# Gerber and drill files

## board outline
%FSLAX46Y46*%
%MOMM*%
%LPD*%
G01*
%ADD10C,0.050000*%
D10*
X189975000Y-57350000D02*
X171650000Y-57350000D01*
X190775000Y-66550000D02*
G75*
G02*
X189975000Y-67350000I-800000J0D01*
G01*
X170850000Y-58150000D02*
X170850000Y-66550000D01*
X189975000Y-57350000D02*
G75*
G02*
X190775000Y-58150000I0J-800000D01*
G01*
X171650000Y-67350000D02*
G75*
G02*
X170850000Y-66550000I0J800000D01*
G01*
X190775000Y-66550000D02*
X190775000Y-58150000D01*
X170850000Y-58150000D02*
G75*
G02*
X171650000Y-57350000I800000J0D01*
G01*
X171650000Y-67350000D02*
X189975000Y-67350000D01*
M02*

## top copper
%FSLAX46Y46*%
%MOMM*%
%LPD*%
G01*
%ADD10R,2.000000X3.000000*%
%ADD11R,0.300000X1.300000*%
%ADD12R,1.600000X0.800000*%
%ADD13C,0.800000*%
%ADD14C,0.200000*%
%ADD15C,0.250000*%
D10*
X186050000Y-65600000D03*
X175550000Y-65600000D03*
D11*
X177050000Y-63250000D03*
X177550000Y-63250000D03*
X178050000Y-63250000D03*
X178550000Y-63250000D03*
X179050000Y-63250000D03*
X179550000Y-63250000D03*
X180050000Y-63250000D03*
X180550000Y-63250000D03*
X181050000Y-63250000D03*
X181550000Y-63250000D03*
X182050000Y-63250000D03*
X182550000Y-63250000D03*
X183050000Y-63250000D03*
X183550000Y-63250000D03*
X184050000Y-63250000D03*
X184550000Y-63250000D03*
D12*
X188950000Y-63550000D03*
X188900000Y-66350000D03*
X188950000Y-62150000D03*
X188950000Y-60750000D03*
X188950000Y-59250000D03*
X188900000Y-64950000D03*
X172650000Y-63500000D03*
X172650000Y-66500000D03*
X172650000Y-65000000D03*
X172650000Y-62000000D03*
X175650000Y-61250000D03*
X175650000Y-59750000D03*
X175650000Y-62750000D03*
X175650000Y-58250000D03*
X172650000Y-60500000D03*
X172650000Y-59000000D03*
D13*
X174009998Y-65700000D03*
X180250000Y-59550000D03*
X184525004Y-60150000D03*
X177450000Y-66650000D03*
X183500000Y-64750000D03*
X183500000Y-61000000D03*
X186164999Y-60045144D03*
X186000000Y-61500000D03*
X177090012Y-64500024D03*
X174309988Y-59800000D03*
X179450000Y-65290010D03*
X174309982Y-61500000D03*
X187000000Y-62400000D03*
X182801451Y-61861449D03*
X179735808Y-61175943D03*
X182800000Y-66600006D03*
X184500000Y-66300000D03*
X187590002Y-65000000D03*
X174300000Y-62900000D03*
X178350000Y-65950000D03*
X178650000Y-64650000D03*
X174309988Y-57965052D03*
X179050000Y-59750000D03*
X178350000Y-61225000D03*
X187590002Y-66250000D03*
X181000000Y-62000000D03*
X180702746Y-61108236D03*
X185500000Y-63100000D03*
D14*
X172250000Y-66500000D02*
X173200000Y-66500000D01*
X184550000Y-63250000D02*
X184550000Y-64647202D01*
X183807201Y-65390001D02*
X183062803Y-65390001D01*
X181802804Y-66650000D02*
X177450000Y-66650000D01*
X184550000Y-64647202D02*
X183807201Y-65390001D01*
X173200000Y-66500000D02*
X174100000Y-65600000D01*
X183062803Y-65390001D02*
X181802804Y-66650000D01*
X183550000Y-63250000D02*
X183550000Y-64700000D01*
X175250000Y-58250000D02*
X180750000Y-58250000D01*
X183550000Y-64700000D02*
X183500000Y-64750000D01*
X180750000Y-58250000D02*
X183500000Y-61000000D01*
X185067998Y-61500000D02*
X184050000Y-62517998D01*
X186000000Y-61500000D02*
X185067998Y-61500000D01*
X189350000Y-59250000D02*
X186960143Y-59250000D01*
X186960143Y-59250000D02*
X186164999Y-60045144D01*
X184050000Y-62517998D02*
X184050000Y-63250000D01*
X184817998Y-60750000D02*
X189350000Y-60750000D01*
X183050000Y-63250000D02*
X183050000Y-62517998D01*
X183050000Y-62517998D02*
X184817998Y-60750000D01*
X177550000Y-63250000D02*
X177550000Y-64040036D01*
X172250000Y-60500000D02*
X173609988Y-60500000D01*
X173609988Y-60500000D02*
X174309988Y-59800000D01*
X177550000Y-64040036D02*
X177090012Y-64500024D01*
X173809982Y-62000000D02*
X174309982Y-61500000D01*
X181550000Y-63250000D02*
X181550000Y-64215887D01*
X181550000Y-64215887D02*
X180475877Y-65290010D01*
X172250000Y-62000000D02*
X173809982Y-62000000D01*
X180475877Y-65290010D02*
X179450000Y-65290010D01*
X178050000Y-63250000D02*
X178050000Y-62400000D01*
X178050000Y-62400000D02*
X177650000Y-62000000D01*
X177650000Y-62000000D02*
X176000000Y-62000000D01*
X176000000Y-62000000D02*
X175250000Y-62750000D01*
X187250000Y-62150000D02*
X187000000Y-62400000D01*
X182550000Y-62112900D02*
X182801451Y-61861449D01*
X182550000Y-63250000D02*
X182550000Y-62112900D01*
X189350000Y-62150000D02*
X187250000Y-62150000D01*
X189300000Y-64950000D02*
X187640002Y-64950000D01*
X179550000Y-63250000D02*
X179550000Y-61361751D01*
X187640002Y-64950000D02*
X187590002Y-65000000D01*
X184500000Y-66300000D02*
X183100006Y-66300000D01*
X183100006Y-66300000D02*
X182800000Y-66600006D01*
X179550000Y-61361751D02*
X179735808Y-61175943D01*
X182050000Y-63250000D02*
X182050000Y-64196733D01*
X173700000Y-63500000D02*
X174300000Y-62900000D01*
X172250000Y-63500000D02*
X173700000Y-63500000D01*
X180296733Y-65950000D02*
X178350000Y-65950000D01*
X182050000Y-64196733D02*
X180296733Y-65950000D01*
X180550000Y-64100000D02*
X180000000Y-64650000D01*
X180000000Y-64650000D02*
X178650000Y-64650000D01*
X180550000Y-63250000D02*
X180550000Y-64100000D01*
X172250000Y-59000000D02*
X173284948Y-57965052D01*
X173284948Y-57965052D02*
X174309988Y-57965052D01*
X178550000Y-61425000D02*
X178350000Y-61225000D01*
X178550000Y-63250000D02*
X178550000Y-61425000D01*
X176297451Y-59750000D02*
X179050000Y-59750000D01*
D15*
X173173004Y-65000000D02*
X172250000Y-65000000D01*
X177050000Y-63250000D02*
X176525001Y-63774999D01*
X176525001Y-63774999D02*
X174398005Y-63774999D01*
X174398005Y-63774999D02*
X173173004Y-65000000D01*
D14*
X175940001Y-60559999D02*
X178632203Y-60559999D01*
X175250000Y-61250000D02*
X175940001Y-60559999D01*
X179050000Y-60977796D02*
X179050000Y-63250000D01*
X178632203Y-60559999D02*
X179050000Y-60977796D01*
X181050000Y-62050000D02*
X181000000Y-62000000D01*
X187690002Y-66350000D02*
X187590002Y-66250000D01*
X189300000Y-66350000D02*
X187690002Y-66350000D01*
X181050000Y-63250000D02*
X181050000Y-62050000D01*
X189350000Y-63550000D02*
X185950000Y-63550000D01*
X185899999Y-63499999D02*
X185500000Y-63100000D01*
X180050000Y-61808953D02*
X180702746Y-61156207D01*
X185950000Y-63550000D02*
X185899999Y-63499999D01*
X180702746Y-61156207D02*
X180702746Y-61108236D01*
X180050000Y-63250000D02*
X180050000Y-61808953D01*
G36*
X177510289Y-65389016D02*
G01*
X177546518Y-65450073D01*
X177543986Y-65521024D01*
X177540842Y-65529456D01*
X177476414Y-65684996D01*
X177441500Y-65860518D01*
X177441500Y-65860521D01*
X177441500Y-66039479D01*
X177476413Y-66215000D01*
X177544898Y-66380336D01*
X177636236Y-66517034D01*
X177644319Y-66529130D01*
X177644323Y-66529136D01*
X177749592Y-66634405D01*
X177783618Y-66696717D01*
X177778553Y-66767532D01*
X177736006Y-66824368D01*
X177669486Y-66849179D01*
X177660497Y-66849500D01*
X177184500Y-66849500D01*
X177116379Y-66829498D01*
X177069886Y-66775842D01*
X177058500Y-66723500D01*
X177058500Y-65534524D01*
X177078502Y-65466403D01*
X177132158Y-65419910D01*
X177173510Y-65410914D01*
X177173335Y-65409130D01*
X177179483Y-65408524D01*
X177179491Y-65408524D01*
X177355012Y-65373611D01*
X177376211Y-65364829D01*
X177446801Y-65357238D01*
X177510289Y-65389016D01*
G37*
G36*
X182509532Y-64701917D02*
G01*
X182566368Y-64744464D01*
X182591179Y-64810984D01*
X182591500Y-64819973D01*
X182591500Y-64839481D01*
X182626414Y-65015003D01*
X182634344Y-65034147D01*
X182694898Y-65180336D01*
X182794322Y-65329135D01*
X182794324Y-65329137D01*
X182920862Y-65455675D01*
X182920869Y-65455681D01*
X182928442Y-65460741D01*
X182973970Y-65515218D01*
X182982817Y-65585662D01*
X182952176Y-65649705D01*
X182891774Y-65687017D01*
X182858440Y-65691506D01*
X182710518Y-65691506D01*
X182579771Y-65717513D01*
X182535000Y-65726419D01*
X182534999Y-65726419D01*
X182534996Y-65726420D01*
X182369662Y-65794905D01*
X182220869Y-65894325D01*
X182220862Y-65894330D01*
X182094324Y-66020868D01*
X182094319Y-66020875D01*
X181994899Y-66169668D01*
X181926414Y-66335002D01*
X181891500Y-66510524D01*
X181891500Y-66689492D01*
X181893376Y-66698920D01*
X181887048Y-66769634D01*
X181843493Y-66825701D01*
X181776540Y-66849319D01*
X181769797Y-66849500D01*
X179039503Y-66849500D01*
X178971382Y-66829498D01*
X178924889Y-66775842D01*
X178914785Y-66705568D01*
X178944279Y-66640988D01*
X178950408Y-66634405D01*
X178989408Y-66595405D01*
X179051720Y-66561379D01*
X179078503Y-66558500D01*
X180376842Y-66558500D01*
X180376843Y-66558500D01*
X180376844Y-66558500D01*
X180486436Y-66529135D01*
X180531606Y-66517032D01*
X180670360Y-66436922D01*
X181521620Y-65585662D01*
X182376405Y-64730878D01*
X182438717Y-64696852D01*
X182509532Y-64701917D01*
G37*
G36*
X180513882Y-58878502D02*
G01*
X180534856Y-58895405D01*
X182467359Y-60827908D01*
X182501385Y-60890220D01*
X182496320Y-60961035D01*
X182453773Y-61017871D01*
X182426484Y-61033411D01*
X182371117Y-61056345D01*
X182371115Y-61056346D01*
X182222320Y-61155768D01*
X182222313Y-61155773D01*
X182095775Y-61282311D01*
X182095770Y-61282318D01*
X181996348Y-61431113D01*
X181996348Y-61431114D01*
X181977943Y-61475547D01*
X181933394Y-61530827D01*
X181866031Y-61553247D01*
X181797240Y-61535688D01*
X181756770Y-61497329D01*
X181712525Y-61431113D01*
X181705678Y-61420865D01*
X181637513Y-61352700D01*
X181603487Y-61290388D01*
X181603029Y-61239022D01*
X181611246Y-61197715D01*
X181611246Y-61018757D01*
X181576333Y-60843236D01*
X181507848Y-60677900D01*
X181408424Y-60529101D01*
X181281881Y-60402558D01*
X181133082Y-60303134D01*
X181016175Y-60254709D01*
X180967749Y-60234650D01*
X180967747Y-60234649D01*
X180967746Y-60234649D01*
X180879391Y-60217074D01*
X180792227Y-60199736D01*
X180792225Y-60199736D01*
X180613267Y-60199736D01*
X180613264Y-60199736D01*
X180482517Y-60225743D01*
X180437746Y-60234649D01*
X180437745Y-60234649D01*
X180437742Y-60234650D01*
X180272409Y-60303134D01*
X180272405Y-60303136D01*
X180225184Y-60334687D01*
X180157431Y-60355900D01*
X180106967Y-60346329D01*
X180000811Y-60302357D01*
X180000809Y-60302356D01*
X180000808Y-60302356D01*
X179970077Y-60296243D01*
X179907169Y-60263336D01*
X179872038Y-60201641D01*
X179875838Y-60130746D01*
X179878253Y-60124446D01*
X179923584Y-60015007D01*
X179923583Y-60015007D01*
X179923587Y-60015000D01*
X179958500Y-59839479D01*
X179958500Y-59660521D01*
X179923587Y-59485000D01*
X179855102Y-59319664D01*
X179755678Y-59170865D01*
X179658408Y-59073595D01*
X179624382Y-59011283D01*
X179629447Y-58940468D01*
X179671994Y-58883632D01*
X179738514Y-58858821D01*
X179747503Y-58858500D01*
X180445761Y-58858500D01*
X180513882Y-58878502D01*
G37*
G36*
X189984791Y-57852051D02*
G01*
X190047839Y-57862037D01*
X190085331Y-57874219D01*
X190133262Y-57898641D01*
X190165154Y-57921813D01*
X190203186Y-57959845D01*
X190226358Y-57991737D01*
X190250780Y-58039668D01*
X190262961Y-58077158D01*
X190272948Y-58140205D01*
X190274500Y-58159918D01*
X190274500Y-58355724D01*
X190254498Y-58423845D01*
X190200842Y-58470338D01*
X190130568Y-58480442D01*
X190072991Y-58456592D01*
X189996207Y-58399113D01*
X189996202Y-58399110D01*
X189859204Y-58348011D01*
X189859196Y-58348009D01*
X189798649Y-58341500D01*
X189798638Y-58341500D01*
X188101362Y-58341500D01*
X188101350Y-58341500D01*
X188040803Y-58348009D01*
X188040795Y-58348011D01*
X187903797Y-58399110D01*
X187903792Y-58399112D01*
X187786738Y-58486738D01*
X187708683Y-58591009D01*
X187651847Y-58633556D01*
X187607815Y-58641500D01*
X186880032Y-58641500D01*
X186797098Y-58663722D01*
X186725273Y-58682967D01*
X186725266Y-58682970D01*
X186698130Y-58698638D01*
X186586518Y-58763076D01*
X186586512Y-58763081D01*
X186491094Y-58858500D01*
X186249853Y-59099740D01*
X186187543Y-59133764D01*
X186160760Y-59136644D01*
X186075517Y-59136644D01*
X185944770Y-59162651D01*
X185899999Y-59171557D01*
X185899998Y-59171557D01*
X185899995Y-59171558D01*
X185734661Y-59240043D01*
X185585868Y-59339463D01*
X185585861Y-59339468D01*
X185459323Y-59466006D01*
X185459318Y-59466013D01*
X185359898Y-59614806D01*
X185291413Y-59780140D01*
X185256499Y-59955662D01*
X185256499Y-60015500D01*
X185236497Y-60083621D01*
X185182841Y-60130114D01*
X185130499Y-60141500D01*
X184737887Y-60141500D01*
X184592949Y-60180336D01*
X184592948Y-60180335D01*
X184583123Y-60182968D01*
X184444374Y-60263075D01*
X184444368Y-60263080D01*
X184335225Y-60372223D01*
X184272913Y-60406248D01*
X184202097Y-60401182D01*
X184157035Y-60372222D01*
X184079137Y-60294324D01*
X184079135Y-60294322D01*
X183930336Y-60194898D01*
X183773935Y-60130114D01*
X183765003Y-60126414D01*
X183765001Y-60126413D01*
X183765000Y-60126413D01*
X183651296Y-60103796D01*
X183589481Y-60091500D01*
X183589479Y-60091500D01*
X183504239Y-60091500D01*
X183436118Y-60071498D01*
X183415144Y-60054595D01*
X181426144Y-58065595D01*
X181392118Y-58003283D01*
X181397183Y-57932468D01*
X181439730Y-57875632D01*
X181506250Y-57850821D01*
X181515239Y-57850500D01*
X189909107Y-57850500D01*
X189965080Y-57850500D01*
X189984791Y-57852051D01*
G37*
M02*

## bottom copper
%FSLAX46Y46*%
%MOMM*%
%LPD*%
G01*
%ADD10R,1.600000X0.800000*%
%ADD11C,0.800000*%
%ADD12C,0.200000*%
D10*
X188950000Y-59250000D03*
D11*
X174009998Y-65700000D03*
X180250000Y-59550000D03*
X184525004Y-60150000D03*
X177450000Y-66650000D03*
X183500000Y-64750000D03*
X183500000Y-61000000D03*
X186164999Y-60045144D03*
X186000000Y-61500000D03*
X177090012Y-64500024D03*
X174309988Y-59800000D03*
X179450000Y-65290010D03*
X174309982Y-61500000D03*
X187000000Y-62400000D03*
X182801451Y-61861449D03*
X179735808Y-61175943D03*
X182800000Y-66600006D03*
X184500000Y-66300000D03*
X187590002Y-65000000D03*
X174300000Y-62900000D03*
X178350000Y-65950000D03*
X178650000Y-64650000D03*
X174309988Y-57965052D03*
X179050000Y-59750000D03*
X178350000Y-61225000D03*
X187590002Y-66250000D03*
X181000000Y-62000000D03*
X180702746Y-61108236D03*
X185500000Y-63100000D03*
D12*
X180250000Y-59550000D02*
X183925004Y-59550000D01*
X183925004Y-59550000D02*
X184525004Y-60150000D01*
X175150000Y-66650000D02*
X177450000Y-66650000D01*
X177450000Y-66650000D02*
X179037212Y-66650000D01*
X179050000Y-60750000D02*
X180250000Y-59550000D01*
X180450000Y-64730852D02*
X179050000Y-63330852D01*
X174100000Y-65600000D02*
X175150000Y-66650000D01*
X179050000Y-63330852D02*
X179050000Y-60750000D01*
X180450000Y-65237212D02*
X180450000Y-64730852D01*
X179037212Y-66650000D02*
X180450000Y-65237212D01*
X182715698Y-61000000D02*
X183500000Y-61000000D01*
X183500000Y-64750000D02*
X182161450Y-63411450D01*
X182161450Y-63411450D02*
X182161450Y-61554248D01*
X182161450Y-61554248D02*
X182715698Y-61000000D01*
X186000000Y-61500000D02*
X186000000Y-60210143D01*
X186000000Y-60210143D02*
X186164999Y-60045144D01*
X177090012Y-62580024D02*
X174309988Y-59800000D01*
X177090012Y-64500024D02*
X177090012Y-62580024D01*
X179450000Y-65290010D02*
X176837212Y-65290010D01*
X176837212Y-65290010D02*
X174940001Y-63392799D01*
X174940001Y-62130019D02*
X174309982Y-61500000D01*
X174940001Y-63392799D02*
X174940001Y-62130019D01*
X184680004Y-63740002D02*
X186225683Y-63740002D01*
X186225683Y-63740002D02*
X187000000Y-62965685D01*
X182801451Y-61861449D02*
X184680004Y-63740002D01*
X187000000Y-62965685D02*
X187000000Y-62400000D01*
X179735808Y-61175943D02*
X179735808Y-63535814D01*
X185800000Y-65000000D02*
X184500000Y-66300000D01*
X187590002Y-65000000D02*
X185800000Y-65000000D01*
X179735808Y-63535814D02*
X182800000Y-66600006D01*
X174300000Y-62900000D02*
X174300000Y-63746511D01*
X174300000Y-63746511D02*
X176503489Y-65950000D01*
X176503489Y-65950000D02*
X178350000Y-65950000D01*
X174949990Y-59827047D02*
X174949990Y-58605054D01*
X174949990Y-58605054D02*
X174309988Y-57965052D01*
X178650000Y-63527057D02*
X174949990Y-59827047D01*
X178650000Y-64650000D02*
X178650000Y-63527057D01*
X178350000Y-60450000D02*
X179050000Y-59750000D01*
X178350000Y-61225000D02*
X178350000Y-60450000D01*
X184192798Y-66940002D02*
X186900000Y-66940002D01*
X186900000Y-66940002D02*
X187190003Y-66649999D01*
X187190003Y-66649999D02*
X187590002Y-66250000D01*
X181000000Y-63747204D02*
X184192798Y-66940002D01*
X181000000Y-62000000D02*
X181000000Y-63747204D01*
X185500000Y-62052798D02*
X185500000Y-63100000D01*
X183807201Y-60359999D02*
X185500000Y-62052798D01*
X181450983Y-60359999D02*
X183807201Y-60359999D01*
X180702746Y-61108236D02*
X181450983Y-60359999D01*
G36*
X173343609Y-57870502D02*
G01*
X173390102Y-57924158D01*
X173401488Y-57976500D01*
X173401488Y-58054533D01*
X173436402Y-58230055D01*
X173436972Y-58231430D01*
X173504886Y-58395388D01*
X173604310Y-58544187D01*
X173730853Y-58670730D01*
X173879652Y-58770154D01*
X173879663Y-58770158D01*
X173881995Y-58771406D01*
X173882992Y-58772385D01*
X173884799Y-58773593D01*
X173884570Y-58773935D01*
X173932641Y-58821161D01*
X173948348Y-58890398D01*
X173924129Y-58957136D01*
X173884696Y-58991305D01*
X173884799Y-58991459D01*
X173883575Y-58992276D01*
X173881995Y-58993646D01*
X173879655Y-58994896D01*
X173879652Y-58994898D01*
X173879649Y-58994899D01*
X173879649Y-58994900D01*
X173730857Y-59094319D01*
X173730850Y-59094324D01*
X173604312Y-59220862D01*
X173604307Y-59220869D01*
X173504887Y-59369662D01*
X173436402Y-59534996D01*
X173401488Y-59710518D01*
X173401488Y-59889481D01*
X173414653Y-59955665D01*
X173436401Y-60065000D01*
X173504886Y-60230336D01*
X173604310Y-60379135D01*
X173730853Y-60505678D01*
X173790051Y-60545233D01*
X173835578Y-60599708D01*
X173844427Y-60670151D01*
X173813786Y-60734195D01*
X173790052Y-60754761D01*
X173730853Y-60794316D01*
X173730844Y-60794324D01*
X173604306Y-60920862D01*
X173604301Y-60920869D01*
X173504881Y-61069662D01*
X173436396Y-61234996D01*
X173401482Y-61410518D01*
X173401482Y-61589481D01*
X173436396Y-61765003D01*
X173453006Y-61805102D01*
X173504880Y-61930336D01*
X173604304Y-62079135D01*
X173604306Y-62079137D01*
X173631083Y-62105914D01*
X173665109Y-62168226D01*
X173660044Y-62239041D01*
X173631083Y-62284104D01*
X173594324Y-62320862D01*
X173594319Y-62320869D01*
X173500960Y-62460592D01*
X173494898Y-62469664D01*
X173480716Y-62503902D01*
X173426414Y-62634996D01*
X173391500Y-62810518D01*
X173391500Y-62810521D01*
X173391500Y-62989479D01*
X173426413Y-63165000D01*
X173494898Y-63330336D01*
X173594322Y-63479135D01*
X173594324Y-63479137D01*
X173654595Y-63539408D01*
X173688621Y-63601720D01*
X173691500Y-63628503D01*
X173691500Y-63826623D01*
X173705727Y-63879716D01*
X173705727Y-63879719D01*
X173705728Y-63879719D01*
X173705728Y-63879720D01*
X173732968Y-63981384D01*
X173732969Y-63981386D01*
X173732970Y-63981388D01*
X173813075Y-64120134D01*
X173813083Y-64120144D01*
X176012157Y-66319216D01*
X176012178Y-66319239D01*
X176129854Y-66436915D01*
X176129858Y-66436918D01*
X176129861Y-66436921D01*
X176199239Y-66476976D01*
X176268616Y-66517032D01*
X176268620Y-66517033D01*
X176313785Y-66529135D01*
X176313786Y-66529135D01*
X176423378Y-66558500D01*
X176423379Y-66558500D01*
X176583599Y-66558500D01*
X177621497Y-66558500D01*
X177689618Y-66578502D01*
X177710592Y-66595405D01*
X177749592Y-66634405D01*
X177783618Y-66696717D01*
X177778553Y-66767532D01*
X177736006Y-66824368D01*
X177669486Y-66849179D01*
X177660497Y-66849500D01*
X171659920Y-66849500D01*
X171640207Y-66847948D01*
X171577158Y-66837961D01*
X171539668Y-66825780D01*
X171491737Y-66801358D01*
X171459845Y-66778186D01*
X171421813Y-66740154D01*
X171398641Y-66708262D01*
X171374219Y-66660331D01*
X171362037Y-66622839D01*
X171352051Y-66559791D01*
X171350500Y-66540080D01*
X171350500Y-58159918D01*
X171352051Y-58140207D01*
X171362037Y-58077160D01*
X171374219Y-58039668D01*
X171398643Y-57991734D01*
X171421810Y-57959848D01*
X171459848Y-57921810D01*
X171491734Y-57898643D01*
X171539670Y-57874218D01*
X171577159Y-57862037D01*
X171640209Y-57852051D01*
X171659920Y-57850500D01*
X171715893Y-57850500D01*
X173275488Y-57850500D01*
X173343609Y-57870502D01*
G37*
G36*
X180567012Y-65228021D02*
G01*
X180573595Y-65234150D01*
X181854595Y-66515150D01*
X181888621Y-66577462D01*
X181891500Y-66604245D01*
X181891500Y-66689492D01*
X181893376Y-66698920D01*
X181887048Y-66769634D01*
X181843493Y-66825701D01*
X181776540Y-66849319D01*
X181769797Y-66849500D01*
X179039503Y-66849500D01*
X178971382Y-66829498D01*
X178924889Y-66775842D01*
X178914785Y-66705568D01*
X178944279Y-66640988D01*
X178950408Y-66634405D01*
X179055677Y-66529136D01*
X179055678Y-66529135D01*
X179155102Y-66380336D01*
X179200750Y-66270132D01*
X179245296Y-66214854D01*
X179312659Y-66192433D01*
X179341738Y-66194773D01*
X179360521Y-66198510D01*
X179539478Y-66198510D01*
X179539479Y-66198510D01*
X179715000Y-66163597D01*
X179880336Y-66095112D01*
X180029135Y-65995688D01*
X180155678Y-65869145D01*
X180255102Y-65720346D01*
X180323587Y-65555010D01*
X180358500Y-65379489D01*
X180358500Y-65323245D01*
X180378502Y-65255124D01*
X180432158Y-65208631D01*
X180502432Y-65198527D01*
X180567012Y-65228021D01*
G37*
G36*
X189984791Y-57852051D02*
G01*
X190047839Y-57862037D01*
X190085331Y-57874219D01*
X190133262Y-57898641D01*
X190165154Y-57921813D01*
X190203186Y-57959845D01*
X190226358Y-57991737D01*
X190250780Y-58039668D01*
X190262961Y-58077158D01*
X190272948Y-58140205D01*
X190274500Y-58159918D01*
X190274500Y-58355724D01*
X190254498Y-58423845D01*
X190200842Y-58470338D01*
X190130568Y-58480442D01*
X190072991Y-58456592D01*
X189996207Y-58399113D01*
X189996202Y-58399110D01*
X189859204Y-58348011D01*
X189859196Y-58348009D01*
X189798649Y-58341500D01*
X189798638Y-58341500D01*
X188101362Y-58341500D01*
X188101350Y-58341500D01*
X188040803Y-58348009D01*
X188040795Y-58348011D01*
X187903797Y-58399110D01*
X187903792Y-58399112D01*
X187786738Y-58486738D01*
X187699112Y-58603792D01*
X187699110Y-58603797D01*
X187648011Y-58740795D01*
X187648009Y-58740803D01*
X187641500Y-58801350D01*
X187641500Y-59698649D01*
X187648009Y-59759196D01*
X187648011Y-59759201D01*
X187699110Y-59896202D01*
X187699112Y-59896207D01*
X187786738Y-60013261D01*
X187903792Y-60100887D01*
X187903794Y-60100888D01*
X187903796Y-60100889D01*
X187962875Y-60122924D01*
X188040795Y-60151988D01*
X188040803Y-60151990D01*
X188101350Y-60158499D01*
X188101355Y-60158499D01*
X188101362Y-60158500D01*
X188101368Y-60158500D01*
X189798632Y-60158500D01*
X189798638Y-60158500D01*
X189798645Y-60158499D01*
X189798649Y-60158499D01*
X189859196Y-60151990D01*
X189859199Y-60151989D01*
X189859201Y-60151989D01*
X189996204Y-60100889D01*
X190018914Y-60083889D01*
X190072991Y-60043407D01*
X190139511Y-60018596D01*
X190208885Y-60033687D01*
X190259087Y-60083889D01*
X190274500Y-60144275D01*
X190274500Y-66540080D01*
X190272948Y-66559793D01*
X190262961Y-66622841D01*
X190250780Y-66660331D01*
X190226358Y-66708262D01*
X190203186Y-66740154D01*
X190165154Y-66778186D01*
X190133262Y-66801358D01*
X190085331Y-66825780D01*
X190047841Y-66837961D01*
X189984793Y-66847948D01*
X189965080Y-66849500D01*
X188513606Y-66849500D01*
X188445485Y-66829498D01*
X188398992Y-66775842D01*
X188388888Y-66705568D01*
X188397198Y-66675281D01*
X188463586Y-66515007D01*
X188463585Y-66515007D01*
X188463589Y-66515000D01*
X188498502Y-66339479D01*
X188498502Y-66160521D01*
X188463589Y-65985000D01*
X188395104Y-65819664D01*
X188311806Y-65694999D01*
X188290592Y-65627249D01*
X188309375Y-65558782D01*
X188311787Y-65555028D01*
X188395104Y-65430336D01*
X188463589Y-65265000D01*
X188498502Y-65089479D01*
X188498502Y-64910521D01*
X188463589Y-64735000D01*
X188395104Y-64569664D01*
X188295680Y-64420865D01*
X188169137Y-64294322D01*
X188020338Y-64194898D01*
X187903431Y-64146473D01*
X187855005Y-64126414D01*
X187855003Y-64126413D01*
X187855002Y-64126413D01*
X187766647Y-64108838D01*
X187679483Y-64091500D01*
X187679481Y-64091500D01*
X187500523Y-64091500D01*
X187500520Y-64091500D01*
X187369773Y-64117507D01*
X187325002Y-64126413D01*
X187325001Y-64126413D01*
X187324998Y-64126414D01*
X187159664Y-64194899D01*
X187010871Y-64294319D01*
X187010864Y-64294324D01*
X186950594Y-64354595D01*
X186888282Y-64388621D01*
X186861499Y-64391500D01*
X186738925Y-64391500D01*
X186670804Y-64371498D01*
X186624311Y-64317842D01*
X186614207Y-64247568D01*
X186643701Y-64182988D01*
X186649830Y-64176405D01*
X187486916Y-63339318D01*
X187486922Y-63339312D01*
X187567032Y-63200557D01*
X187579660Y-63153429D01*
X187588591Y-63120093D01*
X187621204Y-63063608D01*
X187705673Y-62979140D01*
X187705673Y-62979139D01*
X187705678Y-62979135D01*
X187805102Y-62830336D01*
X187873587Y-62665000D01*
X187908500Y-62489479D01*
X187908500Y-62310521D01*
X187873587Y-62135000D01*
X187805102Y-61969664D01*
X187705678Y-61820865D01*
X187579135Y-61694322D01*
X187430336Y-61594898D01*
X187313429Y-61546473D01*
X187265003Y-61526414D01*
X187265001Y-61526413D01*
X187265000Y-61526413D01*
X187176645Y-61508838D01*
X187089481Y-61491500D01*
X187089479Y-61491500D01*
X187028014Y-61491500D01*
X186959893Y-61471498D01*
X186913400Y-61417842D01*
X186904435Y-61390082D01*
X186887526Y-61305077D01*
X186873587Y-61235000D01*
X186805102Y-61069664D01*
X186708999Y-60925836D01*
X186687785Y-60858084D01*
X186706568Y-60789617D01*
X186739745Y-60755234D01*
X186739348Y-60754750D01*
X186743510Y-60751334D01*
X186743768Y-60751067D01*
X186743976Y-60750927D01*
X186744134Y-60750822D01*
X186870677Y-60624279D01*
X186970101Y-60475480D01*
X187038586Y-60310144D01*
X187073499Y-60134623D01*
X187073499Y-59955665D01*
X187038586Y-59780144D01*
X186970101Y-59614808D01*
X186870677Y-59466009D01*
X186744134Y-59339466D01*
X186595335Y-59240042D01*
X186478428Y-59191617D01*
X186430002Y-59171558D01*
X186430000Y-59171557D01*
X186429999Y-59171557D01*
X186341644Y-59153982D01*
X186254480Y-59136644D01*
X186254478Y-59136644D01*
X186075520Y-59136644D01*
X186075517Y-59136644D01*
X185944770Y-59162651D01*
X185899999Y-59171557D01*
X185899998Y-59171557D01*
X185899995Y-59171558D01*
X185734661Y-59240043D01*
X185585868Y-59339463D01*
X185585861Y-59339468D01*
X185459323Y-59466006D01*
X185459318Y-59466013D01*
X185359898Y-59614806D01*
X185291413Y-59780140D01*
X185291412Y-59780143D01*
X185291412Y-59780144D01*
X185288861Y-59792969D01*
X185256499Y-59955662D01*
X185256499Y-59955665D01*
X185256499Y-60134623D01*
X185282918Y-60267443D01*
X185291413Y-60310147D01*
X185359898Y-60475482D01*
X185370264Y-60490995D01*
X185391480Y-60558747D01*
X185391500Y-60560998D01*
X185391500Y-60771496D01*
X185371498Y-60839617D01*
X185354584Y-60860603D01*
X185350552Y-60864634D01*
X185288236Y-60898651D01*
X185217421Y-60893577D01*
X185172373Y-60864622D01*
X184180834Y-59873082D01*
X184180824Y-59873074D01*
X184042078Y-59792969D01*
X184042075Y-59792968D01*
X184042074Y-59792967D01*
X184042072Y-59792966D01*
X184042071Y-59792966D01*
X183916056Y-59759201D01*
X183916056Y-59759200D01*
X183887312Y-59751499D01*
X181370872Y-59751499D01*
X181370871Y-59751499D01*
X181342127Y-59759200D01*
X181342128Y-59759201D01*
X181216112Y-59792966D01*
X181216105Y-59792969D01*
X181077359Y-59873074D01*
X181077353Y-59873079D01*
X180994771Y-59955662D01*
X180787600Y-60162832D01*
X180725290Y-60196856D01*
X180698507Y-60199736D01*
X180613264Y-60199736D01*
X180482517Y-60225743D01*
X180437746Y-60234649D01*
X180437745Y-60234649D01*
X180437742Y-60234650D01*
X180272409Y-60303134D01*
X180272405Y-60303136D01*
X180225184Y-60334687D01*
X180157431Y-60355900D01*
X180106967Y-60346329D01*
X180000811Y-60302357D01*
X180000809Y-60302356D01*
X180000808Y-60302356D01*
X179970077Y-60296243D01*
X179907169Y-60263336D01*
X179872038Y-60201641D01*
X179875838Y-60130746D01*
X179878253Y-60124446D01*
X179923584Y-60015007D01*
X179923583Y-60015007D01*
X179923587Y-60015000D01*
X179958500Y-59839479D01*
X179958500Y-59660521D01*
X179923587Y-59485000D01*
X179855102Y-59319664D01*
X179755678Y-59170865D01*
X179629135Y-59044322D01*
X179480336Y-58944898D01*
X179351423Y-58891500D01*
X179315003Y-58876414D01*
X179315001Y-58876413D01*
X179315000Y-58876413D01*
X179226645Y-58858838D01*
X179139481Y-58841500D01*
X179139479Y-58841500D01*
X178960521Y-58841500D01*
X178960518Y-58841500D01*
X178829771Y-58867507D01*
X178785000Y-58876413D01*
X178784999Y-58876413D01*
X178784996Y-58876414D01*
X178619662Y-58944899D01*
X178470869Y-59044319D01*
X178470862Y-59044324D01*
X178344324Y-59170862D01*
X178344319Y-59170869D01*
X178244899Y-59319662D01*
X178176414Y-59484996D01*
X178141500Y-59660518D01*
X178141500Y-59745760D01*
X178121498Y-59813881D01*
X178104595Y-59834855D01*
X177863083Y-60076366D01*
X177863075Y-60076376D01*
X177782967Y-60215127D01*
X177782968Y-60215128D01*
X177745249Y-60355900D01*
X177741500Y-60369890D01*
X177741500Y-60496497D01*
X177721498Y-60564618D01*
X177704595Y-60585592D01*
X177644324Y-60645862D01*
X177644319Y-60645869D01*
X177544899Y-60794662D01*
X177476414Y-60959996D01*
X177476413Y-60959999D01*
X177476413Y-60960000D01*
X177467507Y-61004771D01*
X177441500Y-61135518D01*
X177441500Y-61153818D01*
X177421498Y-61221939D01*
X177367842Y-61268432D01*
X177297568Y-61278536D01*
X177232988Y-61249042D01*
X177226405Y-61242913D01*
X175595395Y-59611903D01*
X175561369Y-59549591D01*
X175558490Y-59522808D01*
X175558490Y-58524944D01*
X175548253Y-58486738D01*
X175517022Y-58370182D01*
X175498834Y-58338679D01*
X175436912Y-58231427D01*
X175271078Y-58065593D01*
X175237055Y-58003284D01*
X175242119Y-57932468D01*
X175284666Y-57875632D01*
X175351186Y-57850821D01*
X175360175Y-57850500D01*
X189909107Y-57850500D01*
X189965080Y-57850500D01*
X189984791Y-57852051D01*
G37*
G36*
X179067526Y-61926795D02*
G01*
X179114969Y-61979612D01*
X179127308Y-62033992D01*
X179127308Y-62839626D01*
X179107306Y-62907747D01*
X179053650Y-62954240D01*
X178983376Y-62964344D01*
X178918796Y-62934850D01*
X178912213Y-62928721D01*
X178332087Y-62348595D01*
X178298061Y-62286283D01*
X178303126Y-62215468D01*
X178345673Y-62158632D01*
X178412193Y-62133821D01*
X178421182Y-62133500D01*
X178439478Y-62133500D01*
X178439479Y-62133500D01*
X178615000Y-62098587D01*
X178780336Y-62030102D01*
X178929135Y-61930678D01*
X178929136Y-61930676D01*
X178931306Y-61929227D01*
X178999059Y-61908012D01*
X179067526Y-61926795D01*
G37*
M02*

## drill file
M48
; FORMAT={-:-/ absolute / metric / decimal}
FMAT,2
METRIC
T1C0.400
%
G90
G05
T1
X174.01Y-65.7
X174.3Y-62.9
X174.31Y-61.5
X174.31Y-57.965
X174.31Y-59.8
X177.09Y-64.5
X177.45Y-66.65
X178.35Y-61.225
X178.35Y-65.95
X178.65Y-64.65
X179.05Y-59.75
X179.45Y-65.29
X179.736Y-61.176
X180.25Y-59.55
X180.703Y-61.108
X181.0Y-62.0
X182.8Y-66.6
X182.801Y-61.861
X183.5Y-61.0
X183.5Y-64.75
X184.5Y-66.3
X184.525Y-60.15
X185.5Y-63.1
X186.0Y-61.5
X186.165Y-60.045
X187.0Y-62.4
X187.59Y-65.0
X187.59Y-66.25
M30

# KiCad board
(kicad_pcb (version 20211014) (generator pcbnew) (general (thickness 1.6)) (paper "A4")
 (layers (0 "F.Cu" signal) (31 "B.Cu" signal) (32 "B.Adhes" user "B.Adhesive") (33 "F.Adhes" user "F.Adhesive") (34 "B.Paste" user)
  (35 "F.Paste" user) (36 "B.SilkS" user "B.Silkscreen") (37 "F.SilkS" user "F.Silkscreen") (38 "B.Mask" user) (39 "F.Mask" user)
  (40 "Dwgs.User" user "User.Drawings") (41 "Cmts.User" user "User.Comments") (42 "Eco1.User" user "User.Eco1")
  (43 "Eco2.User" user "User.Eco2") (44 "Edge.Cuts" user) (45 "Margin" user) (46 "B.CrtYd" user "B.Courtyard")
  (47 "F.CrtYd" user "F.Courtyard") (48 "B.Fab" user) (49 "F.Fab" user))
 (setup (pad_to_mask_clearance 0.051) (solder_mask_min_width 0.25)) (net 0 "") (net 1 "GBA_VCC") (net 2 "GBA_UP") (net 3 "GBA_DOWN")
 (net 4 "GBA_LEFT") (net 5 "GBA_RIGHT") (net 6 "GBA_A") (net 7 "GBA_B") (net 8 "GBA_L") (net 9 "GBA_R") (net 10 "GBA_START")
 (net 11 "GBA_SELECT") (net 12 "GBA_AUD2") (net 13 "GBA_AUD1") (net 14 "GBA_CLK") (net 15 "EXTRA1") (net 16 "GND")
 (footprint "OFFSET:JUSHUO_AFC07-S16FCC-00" (layer "F.Cu") (at 180.8 65)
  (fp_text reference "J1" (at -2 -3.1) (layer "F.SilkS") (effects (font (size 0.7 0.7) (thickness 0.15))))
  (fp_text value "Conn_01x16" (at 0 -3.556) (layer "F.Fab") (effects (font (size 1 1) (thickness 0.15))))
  (pad "" smd rect locked (at 5.25 0.6) (size 2 3) (layers "F.Cu" "F.Paste" "F.Mask"))
  (pad "" smd rect locked (at -5.25 0.6) (size 2 3) (layers "F.Cu" "F.Paste" "F.Mask"))
  (pad "1" smd rect locked (at -3.75 -1.75) (size 0.3 1.3) (layers "F.Cu" "F.Paste" "F.Mask") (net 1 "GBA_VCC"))
  (pad "2" smd rect locked (at -3.25 -1.75) (size 0.3 1.3) (layers "F.Cu" "F.Paste" "F.Mask") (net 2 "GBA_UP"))
  (pad "3" smd rect locked (at -2.75 -1.75) (size 0.3 1.3) (layers "F.Cu" "F.Paste" "F.Mask") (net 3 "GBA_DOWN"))
  (pad "4" smd rect locked (at -2.25 -1.75) (size 0.3 1.3) (layers "F.Cu" "F.Paste" "F.Mask") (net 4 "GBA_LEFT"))
  (pad "5" smd rect locked (at -1.75 -1.75) (size 0.3 1.3) (layers "F.Cu" "F.Paste" "F.Mask") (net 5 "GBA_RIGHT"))
  (pad "6" smd rect locked (at -1.25 -1.75) (size 0.3 1.3) (layers "F.Cu" "F.Paste" "F.Mask") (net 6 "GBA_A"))
  (pad "7" smd rect locked (at -0.75 -1.75) (size 0.3 1.3) (layers "F.Cu" "F.Paste" "F.Mask") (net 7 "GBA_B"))
  (pad "8" smd rect locked (at -0.25 -1.75) (size 0.3 1.3) (layers "F.Cu" "F.Paste" "F.Mask") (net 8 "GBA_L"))
  (pad "9" smd rect locked (at 0.25 -1.75) (size 0.3 1.3) (layers "F.Cu" "F.Paste" "F.Mask") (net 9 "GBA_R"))
  (pad "10" smd rect locked (at 0.75 -1.75) (size 0.3 1.3) (layers "F.Cu" "F.Paste" "F.Mask") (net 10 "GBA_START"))
  (pad "11" smd rect locked (at 1.25 -1.75) (size 0.3 1.3) (layers "F.Cu" "F.Paste" "F.Mask") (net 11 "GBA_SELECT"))
  (pad "12" smd rect locked (at 1.75 -1.75) (size 0.3 1.3) (layers "F.Cu" "F.Paste" "F.Mask") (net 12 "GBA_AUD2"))
  (pad "13" smd rect locked (at 2.25 -1.75) (size 0.3 1.3) (layers "F.Cu" "F.Paste" "F.Mask") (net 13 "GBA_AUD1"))
  (pad "14" smd rect locked (at 2.75 -1.75) (size 0.3 1.3) (layers "F.Cu" "F.Paste" "F.Mask") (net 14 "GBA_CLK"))
  (pad "15" smd rect locked (at 3.25 -1.75) (size 0.3 1.3) (layers "F.Cu" "F.Paste" "F.Mask") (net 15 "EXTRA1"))
  (pad "16" smd rect locked (at 3.75 -1.75) (size 0.3 1.3) (layers "F.Cu" "F.Paste" "F.Mask") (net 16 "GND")))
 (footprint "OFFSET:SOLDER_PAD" (layer "F.Cu") (at 189.1 63.55 -90)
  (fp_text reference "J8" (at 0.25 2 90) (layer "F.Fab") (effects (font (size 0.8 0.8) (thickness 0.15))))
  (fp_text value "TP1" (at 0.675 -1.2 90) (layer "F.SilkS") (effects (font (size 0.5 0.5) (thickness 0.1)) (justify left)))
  (pad "1" smd rect locked (at 0 -0.25 270) (size 0.8 1.6) (drill (offset 0 0.4)) (layers "F.Cu" "F.Paste" "F.Mask") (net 7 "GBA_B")))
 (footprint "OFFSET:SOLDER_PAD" (layer "F.Cu") (at 189.05 66.35 -90)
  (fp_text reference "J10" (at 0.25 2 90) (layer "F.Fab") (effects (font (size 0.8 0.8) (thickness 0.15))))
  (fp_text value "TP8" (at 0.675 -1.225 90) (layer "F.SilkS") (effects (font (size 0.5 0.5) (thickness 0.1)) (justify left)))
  (pad "1" smd rect locked (at 0 -0.25 270) (size 0.8 1.6) (drill (offset 0 0.4)) (layers "F.Cu" "F.Paste" "F.Mask") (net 9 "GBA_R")))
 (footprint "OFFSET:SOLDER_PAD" (layer "F.Cu") (at 189.1 62.15 -90)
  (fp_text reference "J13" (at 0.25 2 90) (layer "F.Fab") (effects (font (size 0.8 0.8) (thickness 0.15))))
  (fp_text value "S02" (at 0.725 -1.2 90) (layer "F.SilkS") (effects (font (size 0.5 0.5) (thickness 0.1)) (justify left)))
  (pad "1" smd rect locked (at 0 -0.25 270) (size 0.8 1.6) (drill (offset 0 0.4)) (layers "F.Cu" "F.Paste" "F.Mask") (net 12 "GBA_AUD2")))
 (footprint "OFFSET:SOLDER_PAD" (layer "F.Cu") (at 189.1 60.75 -90)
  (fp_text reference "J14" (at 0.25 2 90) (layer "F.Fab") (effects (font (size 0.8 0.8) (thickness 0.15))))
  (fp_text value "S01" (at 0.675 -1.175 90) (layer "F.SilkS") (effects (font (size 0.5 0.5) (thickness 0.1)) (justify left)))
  (pad "1" smd rect locked (at 0 -0.25 270) (size 0.8 1.6) (drill (offset 0 0.4)) (layers "F.Cu" "F.Paste" "F.Mask") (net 13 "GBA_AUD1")))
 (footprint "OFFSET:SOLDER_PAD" (layer "F.Cu") (at 189.1 59.25 -90)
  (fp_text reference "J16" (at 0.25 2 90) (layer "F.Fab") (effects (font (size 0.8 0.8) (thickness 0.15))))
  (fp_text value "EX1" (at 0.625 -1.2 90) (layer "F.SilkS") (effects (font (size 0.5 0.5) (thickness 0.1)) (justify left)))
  (pad "1" smd rect locked (at 0 -0.25 270) (size 0.8 1.6) (drill (offset 0 0.4)) (layers "F.Cu" "F.Paste" "F.Mask") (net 15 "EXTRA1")))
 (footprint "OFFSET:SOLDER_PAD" (layer "F.Cu") (at 189.05 64.95 -90)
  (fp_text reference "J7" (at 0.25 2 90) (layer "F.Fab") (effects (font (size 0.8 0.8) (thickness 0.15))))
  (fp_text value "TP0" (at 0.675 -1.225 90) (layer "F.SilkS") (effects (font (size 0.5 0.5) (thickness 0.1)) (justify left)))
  (pad "1" smd rect locked (at 0 -0.25 270) (size 0.8 1.6) (drill (offset 0 0.4)) (layers "F.Cu" "F.Paste" "F.Mask") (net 6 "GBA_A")))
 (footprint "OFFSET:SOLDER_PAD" (layer "F.Cu") (at 172.5 63.5 90)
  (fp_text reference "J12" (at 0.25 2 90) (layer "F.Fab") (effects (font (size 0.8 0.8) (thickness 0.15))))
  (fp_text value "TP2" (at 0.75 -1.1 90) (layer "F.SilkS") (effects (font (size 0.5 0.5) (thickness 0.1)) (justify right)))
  (pad "1" smd rect locked (at 0 -0.25 90) (size 0.8 1.6) (drill (offset 0 0.4)) (layers "F.Cu" "F.Paste" "F.Mask") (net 11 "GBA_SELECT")))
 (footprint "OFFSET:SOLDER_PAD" (layer "F.Cu") (at 172.5 66.5 90)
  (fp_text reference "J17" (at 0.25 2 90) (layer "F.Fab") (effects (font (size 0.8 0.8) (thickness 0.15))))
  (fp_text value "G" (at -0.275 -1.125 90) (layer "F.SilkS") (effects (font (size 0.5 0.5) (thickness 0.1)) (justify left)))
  (pad "1" smd rect locked (at 0 -0.25 90) (size 0.8 1.6) (drill (offset 0 0.4)) (layers "F.Cu" "F.Paste" "F.Mask") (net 16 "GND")))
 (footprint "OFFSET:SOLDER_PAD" (layer "F.Cu") (at 172.5 65 90)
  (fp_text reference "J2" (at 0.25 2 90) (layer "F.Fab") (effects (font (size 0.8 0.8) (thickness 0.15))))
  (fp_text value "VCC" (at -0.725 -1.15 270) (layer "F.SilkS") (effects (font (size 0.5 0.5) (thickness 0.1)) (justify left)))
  (pad "1" smd rect locked (at 0 -0.25 90) (size 0.8 1.6) (drill (offset 0 0.4)) (layers "F.Cu" "F.Paste" "F.Mask") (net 1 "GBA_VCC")))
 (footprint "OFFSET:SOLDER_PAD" (layer "F.Cu") (at 172.5 62 90)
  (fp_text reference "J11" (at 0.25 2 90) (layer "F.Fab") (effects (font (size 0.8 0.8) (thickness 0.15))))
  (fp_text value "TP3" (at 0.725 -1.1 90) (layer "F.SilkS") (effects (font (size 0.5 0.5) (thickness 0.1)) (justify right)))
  (pad "1" smd rect locked (at 0 -0.25 90) (size 0.8 1.6) (drill (offset 0 0.4)) (layers "F.Cu" "F.Paste" "F.Mask") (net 10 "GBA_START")))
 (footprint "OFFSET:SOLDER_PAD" (layer "F.Cu") (at 175.5 61.25 90)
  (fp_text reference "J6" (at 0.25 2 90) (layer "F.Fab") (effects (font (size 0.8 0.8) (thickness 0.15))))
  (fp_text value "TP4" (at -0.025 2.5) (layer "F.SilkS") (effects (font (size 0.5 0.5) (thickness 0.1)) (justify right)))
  (pad "1" smd rect locked (at 0 -0.25 90) (size 0.8 1.6) (drill (offset 0 0.4)) (layers "F.Cu" "F.Paste" "F.Mask") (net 5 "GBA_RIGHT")))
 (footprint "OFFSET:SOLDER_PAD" (layer "F.Cu") (at 175.5 59.75 90)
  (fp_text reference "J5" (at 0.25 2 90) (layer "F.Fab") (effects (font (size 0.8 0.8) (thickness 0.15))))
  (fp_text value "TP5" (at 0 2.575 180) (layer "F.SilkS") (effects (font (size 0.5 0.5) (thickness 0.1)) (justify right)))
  (pad "1" smd rect locked (at 0 -0.25 90) (size 0.8 1.6) (drill (offset 0 0.4)) (layers "F.Cu" "F.Paste" "F.Mask") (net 4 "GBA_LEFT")))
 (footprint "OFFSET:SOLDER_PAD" (layer "F.Cu") (at 175.5 62.75 90)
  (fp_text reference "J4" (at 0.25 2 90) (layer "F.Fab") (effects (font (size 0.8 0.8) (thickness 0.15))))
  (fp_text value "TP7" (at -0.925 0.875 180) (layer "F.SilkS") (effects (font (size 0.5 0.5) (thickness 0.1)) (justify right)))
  (pad "1" smd rect locked (at 0 -0.25 90) (size 0.8 1.6) (drill (offset 0 0.4)) (layers "F.Cu" "F.Paste" "F.Mask") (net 3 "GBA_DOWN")))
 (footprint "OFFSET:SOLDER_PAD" (layer "F.Cu") (at 175.5 58.25 90)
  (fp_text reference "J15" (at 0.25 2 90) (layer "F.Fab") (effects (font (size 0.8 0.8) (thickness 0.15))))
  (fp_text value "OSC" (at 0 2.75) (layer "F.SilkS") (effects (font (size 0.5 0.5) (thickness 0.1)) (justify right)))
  (pad "1" smd rect locked (at 0 -0.25 90) (size 0.8 1.6) (drill (offset 0 0.4)) (layers "F.Cu" "F.Paste" "F.Mask") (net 14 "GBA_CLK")))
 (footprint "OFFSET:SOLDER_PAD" (layer "F.Cu") (at 172.5 60.5 90)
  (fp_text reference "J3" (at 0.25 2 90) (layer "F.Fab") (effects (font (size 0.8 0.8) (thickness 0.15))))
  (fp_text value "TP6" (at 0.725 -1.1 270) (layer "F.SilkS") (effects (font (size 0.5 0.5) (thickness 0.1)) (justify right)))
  (pad "1" smd rect locked (at 0 -0.25 90) (size 0.8 1.6) (drill (offset 0 0.4)) (layers "F.Cu" "F.Paste" "F.Mask") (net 2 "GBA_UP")))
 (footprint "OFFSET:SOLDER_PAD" (layer "F.Cu") (at 172.5 59 90)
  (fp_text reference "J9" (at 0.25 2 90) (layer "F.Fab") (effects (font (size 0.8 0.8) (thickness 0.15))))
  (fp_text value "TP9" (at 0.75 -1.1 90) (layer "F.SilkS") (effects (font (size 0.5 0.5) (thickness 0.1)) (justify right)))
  (pad "1" smd rect locked (at 0 -0.25 90) (size 0.8 1.6) (drill (offset 0 0.4)) (layers "F.Cu" "F.Paste" "F.Mask") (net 8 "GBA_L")))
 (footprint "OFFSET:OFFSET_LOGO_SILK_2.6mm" (layer "B.Cu") (at 180.575 62.275 180)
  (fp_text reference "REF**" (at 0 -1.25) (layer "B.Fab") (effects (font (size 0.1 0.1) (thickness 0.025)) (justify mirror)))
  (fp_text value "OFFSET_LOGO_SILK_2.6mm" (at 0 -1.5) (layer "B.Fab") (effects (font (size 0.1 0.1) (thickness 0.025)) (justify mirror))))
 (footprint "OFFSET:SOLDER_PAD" (layer "B.Cu") (at 188.8 59.25 -90)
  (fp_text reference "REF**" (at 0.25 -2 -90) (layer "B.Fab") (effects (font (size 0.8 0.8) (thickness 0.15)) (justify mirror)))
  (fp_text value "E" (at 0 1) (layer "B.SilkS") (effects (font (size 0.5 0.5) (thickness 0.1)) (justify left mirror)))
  (pad "1" smd rect locked (at 0 0.25 270) (size 0.8 1.6) (drill (offset 0 -0.4)) (layers "B.Cu" "B.Paste" "B.Mask")))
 (gr_line (start 189.975 57.35) (end 171.65 57.35) (layer "Edge.Cuts") (width 0.05))
 (gr_arc (start 190.775 66.55) (mid 190.540685 67.115685) (end 189.975 67.35) (layer "Edge.Cuts") (width 0.05))
 (gr_line (start 170.85 58.15) (end 170.85 66.55) (layer "Edge.Cuts") (width 0.05))
 (gr_arc (start 189.975 57.35) (mid 190.540685 57.584315) (end 190.775 58.15) (layer "Edge.Cuts") (width 0.05))
 (gr_arc (start 171.65 67.35) (mid 171.084315 67.115685) (end 170.85 66.55) (layer "Edge.Cuts") (width 0.05))
 (gr_line (start 190.775 66.55) (end 190.775 58.15) (layer "Edge.Cuts") (width 0.05))
 (gr_arc (start 170.85 58.15) (mid 171.084315 57.584315) (end 171.65 57.35) (layer "Edge.Cuts") (width 0.05))
 (gr_line (start 171.65 67.35) (end 189.975 67.35) (layer "Edge.Cuts") (width 0.05))
 (segment (start 172.25 66.5) (end 173.2 66.5) (width 0.2) (layer "F.Cu") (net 16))
 (segment (start 184.55 63.25) (end 184.55 64.647202) (width 0.2) (layer "F.Cu") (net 16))
 (segment (start 183.807201 65.390001) (end 183.062803 65.390001) (width 0.2) (layer "F.Cu") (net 16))
 (segment (start 181.802804 66.65) (end 177.45 66.65) (width 0.2) (layer "F.Cu") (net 16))
 (segment (start 184.55 64.647202) (end 183.807201 65.390001) (width 0.2) (layer "F.Cu") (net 16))
 (segment (start 173.2 66.5) (end 174.1 65.6) (width 0.2) (layer "F.Cu") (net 16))
 (segment (start 183.062803 65.390001) (end 181.802804 66.65) (width 0.2) (layer "F.Cu") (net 16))
 (via (at 174.009998 65.7) (size 0.8) (drill 0.4) (layers "F.Cu" "B.Cu") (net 16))
 (via (at 180.25 59.55) (size 0.8) (drill 0.4) (layers "F.Cu" "B.Cu") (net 16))
 (via (at 184.525004 60.15) (size 0.8) (drill 0.4) (layers "F.Cu" "B.Cu") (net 16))
 (via (at 177.45 66.65) (size 0.8) (drill 0.4) (layers "F.Cu" "B.Cu") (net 16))
 (segment (start 180.25 59.55) (end 183.925004 59.55) (width 0.2) (layer "B.Cu") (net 16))
 (segment (start 183.925004 59.55) (end 184.525004 60.15) (width 0.2) (layer "B.Cu") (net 16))
 (segment (start 175.15 66.65) (end 177.45 66.65) (width 0.2) (layer "B.Cu") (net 16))
 (segment (start 177.45 66.65) (end 179.037212 66.65) (width 0.2) (layer "B.Cu") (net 16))
 (segment (start 179.05 60.75) (end 180.25 59.55) (width 0.2) (layer "B.Cu") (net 16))
 (segment (start 180.45 64.730852) (end 179.05 63.330852) (width 0.2) (layer "B.Cu") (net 16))
 (segment (start 174.1 65.6) (end 175.15 66.65) (width 0.2) (layer "B.Cu") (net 16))
 (segment (start 179.05 63.330852) (end 179.05 60.75) (width 0.2) (layer "B.Cu") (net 16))
 (segment (start 180.45 65.237212) (end 180.45 64.730852) (width 0.2) (layer "B.Cu") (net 16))
 (segment (start 179.037212 66.65) (end 180.45 65.237212) (width 0.2) (layer "B.Cu") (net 16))
 (segment (start 183.55 63.25) (end 183.55 64.7) (width 0.2) (layer "F.Cu") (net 14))
 (segment (start 175.25 58.25) (end 180.75 58.25) (width 0.2) (layer "F.Cu") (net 14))
 (segment (start 183.55 64.7) (end 183.5 64.75) (width 0.2) (layer "F.Cu") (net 14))
 (segment (start 180.75 58.25) (end 183.5 61) (width 0.2) (layer "F.Cu") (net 14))
 (via (at 183.5 64.75) (size 0.8) (drill 0.4) (layers "F.Cu" "B.Cu") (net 14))
 (via (at 183.5 61) (size 0.8) (drill 0.4) (layers "F.Cu" "B.Cu") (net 14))
 (segment (start 182.715698 61) (end 183.5 61) (width 0.2) (layer "B.Cu") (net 14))
 (segment (start 183.5 64.75) (end 182.16145 63.41145) (width 0.2) (layer "B.Cu") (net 14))
 (segment (start 182.16145 63.41145) (end 182.16145 61.554248) (width 0.2) (layer "B.Cu") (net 14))
 (segment (start 182.16145 61.554248) (end 182.715698 61) (width 0.2) (layer "B.Cu") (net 14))
 (segment (start 185.067998 61.5) (end 184.05 62.517998) (width 0.2) (layer "F.Cu") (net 15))
 (segment (start 186 61.5) (end 185.067998 61.5) (width 0.2) (layer "F.Cu") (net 15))
 (segment (start 189.35 59.25) (end 186.960143 59.25) (width 0.2) (layer "F.Cu") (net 15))
 (segment (start 186.960143 59.25) (end 186.164999 60.045144) (width 0.2) (layer "F.Cu") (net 15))
 (segment (start 184.05 62.517998) (end 184.05 63.25) (width 0.2) (layer "F.Cu") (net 15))
 (via (at 186.164999 60.045144) (size 0.8) (drill 0.4) (layers "F.Cu" "B.Cu") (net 15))
 (via (at 186 61.5) (size 0.8) (drill 0.4) (layers "F.Cu" "B.Cu") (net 15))
 (segment (start 186 61.5) (end 186 60.210143) (width 0.2) (layer "B.Cu") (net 15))
 (segment (start 186 60.210143) (end 186.164999 60.045144) (width 0.2) (layer "B.Cu") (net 15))
 (segment (start 184.817998 60.75) (end 189.35 60.75) (width 0.2) (layer "F.Cu") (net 13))
 (segment (start 183.05 63.25) (end 183.05 62.517998) (width 0.2) (layer "F.Cu") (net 13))
 (segment (start 183.05 62.517998) (end 184.817998 60.75) (width 0.2) (layer "F.Cu") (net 13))
 (segment (start 177.55 63.25) (end 177.55 64.040036) (width 0.2) (layer "F.Cu") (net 2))
 (segment (start 172.25 60.5) (end 173.609988 60.5) (width 0.2) (layer "F.Cu") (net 2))
 (segment (start 173.609988 60.5) (end 174.309988 59.8) (width 0.2) (layer "F.Cu") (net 2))
 (segment (start 177.55 64.040036) (end 177.090012 64.500024) (width 0.2) (layer "F.Cu") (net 2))
 (via (at 177.090012 64.500024) (size 0.8) (drill 0.4) (layers "F.Cu" "B.Cu") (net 2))
 (via (at 174.309988 59.8) (size 0.8) (drill 0.4) (layers "F.Cu" "B.Cu") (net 2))
 (segment (start 177.090012 62.580024) (end 174.309988 59.8) (width 0.2) (layer "B.Cu") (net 2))
 (segment (start 177.090012 64.500024) (end 177.090012 62.580024) (width 0.2) (layer "B.Cu") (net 2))
 (segment (start 173.809982 62) (end 174.309982 61.5) (width 0.2) (layer "F.Cu") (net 10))
 (segment (start 181.55 63.25) (end 181.55 64.215887) (width 0.2) (layer "F.Cu") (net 10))
 (segment (start 181.55 64.215887) (end 180.475877 65.29001) (width 0.2) (layer "F.Cu") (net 10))
 (segment (start 172.25 62) (end 173.809982 62) (width 0.2) (layer "F.Cu") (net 10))
 (segment (start 180.475877 65.29001) (end 179.45 65.29001) (width 0.2) (layer "F.Cu") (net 10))
 (via (at 179.45 65.29001) (size 0.8) (drill 0.4) (layers "F.Cu" "B.Cu") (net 10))
 (via (at 174.309982 61.5) (size 0.8) (drill 0.4) (layers "F.Cu" "B.Cu") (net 10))
 (segment (start 179.45 65.29001) (end 176.837212 65.29001) (width 0.2) (layer "B.Cu") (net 10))
 (segment (start 176.837212 65.29001) (end 174.940001 63.392799) (width 0.2) (layer "B.Cu") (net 10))
 (segment (start 174.940001 62.130019) (end 174.309982 61.5) (width 0.2) (layer "B.Cu") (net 10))
 (segment (start 174.940001 63.392799) (end 174.940001 62.130019) (width 0.2) (layer "B.Cu") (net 10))
 (segment (start 178.05 63.25) (end 178.05 62.4) (width 0.2) (layer "F.Cu") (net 3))
 (segment (start 178.05 62.4) (end 177.65 62) (width 0.2) (layer "F.Cu") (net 3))
 (segment (start 177.65 62) (end 176 62) (width 0.2) (layer "F.Cu") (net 3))
 (segment (start 176 62) (end 175.25 62.75) (width 0.2) (layer "F.Cu") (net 3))
 (segment (start 187.25 62.15) (end 187 62.4) (width 0.2) (layer "F.Cu") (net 12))
 (segment (start 182.55 62.1129) (end 182.801451 61.861449) (width 0.2) (layer "F.Cu") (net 12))
 (segment (start 182.55 63.25) (end 182.55 62.1129) (width 0.2) (layer "F.Cu") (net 12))
 (segment (start 189.35 62.15) (end 187.25 62.15) (width 0.2) (layer "F.Cu") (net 12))
 (via (at 187 62.4) (size 0.8) (drill 0.4) (layers "F.Cu" "B.Cu") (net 12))
 (via (at 182.801451 61.861449) (size 0.8) (drill 0.4) (layers "F.Cu" "B.Cu") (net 12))
 (segment (start 184.680004 63.740002) (end 186.225683 63.740002) (width 0.2) (layer "B.Cu") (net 12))
 (segment (start 186.225683 63.740002) (end 187 62.965685) (width 0.2) (layer "B.Cu") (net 12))
 (segment (start 182.801451 61.861449) (end 184.680004 63.740002) (width 0.2) (layer "B.Cu") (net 12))
 (segment (start 187 62.965685) (end 187 62.4) (width 0.2) (layer "B.Cu") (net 12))
 (segment (start 189.3 64.95) (end 187.640002 64.95) (width 0.2) (layer "F.Cu") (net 6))
 (segment (start 179.55 63.25) (end 179.55 61.361751) (width 0.2) (layer "F.Cu") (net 6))
 (segment (start 187.640002 64.95) (end 187.590002 65) (width 0.2) (layer "F.Cu") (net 6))
 (segment (start 184.5 66.3) (end 183.100006 66.3) (width 0.2) (layer "F.Cu") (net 6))
 (segment (start 183.100006 66.3) (end 182.8 66.600006) (width 0.2) (layer "F.Cu") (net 6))
 (segment (start 179.55 61.361751) (end 179.735808 61.175943) (width 0.2) (layer "F.Cu") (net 6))
 (via (at 179.735808 61.175943) (size 0.8) (drill 0.4) (layers "F.Cu" "B.Cu") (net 6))
 (via (at 182.8 66.600006) (size 0.8) (drill 0.4) (layers "F.Cu" "B.Cu") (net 6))
 (via (at 184.5 66.3) (size 0.8) (drill 0.4) (layers "F.Cu" "B.Cu") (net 6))
 (via (at 187.590002 65) (size 0.8) (drill 0.4) (layers "F.Cu" "B.Cu") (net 6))
 (segment (start 179.735808 61.175943) (end 179.735808 63.535814) (width 0.2) (layer "B.Cu") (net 6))
 (segment (start 185.8 65) (end 184.5 66.3) (width 0.2) (layer "B.Cu") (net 6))
 (segment (start 187.590002 65) (end 185.8 65) (width 0.2) (layer "B.Cu") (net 6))
 (segment (start 179.735808 63.535814) (end 182.8 66.600006) (width 0.2) (layer "B.Cu") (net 6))
 (segment (start 182.05 63.25) (end 182.05 64.196733) (width 0.2) (layer "F.Cu") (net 11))
 (segment (start 173.7 63.5) (end 174.3 62.9) (width 0.2) (layer "F.Cu") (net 11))
 (segment (start 172.25 63.5) (end 173.7 63.5) (width 0.2) (layer "F.Cu") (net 11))
 (segment (start 180.296733 65.95) (end 178.35 65.95) (width 0.2) (layer "F.Cu") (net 11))
 (segment (start 182.05 64.196733) (end 180.296733 65.95) (width 0.2) (layer "F.Cu") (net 11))
 (via (at 174.3 62.9) (size 0.8) (drill 0.4) (layers "F.Cu" "B.Cu") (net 11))
 (via (at 178.35 65.95) (size 0.8) (drill 0.4) (layers "F.Cu" "B.Cu") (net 11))
 (segment (start 174.3 62.9) (end 174.3 63.746511) (width 0.2) (layer "B.Cu") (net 11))
 (segment (start 174.3 63.746511) (end 176.503489 65.95) (width 0.2) (layer "B.Cu") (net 11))
 (segment (start 176.503489 65.95) (end 178.35 65.95) (width 0.2) (layer "B.Cu") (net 11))
 (segment (start 180.55 64.1) (end 180 64.65) (width 0.2) (layer "F.Cu") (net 8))
 (segment (start 180 64.65) (end 178.65 64.65) (width 0.2) (layer "F.Cu") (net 8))
 (segment (start 180.55 63.25) (end 180.55 64.1) (width 0.2) (layer "F.Cu") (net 8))
 (segment (start 172.25 59) (end 173.284948 57.965052) (width 0.2) (layer "F.Cu") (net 8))
 (segment (start 173.284948 57.965052) (end 174.309988 57.965052) (width 0.2) (layer "F.Cu") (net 8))
 (via (at 178.65 64.65) (size 0.8) (drill 0.4) (layers "F.Cu" "B.Cu") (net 8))
 (via (at 174.309988 57.965052) (size 0.8) (drill 0.4) (layers "F.Cu" "B.Cu") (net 8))
 (segment (start 174.94999 59.827047) (end 174.94999 58.605054) (width 0.2) (layer "B.Cu") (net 8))
 (segment (start 174.94999 58.605054) (end 174.309988 57.965052) (width 0.2) (layer "B.Cu") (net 8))
 (segment (start 178.65 63.527057) (end 174.94999 59.827047) (width 0.2) (layer "B.Cu") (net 8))
 (segment (start 178.65 64.65) (end 178.65 63.527057) (width 0.2) (layer "B.Cu") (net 8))
 (segment (start 178.55 61.425) (end 178.35 61.225) (width 0.2) (layer "F.Cu") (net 4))
 (segment (start 178.55 63.25) (end 178.55 61.425) (width 0.2) (layer "F.Cu") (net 4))
 (segment (start 176.297451 59.75) (end 179.05 59.75) (width 0.2) (layer "F.Cu") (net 4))
 (via (at 179.05 59.75) (size 0.8) (drill 0.4) (layers "F.Cu" "B.Cu") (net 4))
 (via (at 178.35 61.225) (size 0.8) (drill 0.4) (layers "F.Cu" "B.Cu") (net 4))
 (segment (start 178.35 60.45) (end 179.05 59.75) (width 0.2) (layer "B.Cu") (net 4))
 (segment (start 178.35 61.225) (end 178.35 60.45) (width 0.2) (layer "B.Cu") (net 4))
 (segment (start 173.173004 65) (end 172.25 65) (width 0.25) (layer "F.Cu") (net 1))
 (segment (start 177.05 63.25) (end 176.525001 63.774999) (width 0.25) (layer "F.Cu") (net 1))
 (segment (start 176.525001 63.774999) (end 174.398005 63.774999) (width 0.25) (layer "F.Cu") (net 1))
 (segment (start 174.398005 63.774999) (end 173.173004 65) (width 0.25) (layer "F.Cu") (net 1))
 (segment (start 175.940001 60.559999) (end 178.632203 60.559999) (width 0.2) (layer "F.Cu") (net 5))
 (segment (start 175.25 61.25) (end 175.940001 60.559999) (width 0.2) (layer "F.Cu") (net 5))
 (segment (start 179.05 60.977796) (end 179.05 63.25) (width 0.2) (layer "F.Cu") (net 5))
 (segment (start 178.632203 60.559999) (end 179.05 60.977796) (width 0.2) (layer "F.Cu") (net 5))
 (segment (start 181.05 62.05) (end 181 62) (width 0.2) (layer "F.Cu") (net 9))
 (segment (start 187.690002 66.35) (end 187.590002 66.25) (width 0.2) (layer "F.Cu") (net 9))
 (segment (start 189.3 66.35) (end 187.690002 66.35) (width 0.2) (layer "F.Cu") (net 9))
 (segment (start 181.05 63.25) (end 181.05 62.05) (width 0.2) (layer "F.Cu") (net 9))
 (via (at 187.590002 66.25) (size 0.8) (drill 0.4) (layers "F.Cu" "B.Cu") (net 9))
 (via (at 181 62) (size 0.8) (drill 0.4) (layers "F.Cu" "B.Cu") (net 9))
 (segment (start 184.192798 66.940002) (end 186.9 66.940002) (width 0.2) (layer "B.Cu") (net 9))
 (segment (start 186.9 66.940002) (end 187.190003 66.649999) (width 0.2) (layer "B.Cu") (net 9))
 (segment (start 187.190003 66.649999) (end 187.590002 66.25) (width 0.2) (layer "B.Cu") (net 9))
 (segment (start 181 63.747204) (end 184.192798 66.940002) (width 0.2) (layer "B.Cu") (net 9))
 (segment (start 181 62) (end 181 63.747204) (width 0.2) (layer "B.Cu") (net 9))
 (segment (start 189.35 63.55) (end 185.95 63.55) (width 0.2) (layer "F.Cu") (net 7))
 (segment (start 185.899999 63.499999) (end 185.5 63.1) (width 0.2) (layer "F.Cu") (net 7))
 (segment (start 180.05 61.808953) (end 180.702746 61.156207) (width 0.2) (layer "F.Cu") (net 7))
 (segment (start 185.95 63.55) (end 185.899999 63.499999) (width 0.2) (layer "F.Cu") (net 7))
 (segment (start 180.702746 61.156207) (end 180.702746 61.108236) (width 0.2) (layer "F.Cu") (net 7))
 (segment (start 180.05 63.25) (end 180.05 61.808953) (width 0.2) (layer "F.Cu") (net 7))
 (via (at 180.702746 61.108236) (size 0.8) (drill 0.4) (layers "F.Cu" "B.Cu") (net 7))
 (via (at 185.5 63.1) (size 0.8) (drill 0.4) (layers "F.Cu" "B.Cu") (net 7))
 (segment (start 185.5 62.052798) (end 185.5 63.1) (width 0.2) (layer "B.Cu") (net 7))
 (segment (start 183.807201 60.359999) (end 185.5 62.052798) (width 0.2) (layer "B.Cu") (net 7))
 (segment (start 181.450983 60.359999) (end 183.807201 60.359999) (width 0.2) (layer "B.Cu") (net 7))
 (segment (start 180.702746 61.108236) (end 181.450983 60.359999) (width 0.2) (layer "B.Cu") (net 7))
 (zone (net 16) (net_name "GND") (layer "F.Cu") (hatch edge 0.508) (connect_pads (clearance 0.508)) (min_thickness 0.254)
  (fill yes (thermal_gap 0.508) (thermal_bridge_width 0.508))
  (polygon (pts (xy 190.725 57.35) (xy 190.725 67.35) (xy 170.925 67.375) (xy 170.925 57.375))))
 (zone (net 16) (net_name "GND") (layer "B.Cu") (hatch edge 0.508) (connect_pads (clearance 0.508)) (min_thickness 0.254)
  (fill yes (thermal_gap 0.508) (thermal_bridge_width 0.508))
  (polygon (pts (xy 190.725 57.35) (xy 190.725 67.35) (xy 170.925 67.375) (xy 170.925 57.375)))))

